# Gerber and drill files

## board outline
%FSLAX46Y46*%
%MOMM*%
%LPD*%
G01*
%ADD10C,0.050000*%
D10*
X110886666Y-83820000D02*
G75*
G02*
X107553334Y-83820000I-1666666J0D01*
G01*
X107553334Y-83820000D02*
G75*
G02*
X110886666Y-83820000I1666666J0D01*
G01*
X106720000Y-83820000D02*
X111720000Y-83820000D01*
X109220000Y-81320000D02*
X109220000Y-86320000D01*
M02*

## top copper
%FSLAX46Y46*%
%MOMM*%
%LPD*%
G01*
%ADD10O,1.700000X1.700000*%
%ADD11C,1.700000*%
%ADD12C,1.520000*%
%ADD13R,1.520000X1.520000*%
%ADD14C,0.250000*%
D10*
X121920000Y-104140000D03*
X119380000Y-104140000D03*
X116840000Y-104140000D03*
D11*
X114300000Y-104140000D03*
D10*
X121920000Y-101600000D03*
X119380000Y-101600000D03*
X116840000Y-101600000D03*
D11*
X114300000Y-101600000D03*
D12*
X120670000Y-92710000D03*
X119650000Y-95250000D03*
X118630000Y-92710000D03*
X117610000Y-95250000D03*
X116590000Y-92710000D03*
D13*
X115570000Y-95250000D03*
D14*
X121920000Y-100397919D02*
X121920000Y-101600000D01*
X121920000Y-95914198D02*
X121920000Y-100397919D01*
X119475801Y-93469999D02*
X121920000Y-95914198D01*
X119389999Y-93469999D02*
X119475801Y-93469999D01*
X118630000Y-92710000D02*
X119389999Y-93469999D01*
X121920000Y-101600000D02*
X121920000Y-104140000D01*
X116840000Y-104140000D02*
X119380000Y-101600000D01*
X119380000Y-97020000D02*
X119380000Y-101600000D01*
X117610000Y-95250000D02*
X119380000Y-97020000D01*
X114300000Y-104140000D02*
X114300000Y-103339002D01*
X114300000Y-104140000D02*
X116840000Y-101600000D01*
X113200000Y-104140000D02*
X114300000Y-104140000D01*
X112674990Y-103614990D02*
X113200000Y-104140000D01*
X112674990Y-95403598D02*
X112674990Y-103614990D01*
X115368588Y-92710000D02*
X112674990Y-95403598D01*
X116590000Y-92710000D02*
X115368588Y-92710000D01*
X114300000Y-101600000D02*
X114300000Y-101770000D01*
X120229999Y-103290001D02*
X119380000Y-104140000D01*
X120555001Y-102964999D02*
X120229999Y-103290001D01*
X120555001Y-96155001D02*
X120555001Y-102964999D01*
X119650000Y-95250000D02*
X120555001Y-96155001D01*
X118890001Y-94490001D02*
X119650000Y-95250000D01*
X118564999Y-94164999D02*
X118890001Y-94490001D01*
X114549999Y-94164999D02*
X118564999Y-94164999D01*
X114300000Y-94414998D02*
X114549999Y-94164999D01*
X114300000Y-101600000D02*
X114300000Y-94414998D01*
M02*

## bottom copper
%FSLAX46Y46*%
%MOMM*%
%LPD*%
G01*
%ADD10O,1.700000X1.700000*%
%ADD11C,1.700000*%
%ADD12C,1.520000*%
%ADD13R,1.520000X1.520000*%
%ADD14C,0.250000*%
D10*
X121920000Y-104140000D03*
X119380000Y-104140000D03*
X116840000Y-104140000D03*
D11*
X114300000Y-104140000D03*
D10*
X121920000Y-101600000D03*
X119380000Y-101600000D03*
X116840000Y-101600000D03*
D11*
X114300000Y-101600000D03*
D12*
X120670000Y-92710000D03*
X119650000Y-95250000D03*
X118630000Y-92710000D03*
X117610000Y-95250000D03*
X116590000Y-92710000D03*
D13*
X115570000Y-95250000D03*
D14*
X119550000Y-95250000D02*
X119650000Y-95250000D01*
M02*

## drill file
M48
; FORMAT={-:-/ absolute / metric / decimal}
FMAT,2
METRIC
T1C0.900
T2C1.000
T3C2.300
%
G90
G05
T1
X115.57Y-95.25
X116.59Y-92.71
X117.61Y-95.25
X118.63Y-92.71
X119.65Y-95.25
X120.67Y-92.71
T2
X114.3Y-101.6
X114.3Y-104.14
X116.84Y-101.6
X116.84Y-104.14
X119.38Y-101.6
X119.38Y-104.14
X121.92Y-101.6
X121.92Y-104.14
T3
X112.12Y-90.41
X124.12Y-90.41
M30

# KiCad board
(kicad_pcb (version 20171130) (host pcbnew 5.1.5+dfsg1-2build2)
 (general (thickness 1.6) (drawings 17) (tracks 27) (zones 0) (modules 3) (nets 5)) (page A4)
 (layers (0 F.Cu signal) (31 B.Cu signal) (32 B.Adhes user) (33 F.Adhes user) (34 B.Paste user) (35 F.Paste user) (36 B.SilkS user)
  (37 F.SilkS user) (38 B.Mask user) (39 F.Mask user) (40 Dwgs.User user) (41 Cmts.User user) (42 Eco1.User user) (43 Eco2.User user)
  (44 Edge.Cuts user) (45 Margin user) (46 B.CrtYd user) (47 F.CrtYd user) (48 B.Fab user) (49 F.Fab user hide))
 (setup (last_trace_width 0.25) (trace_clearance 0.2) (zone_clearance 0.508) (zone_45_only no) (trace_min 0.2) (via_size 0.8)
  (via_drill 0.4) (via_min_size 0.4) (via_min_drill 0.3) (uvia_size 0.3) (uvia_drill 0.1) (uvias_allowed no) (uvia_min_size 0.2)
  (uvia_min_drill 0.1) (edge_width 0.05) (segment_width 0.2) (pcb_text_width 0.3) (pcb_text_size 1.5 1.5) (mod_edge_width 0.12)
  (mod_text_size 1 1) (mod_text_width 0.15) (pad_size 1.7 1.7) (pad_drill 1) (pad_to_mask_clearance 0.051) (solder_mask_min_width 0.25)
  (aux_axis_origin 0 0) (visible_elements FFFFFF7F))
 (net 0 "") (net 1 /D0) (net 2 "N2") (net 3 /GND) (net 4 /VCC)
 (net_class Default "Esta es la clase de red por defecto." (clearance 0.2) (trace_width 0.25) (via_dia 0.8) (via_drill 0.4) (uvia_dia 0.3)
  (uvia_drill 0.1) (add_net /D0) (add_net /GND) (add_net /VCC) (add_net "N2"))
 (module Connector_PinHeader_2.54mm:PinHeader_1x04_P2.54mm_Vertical (layer F.Cu) (at 114.3 104.14 90)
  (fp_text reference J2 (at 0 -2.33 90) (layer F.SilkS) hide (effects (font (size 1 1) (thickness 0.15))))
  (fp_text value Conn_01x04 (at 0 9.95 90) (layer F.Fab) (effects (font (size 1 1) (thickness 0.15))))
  (pad 4 thru_hole oval (at 0 7.62 90) (size 1.7 1.7) (drill 1) (layers *.Cu *.Mask) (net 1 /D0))
  (pad 3 thru_hole oval (at 0 5.08 90) (size 1.7 1.7) (drill 1) (layers *.Cu *.Mask) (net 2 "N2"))
  (pad 2 thru_hole oval (at 0 2.54 90) (size 1.7 1.7) (drill 1) (layers *.Cu *.Mask) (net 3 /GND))
  (pad 1 thru_hole circle (at 0 0 90) (size 1.7 1.7) (drill 1) (layers *.Cu *.Mask) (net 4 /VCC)))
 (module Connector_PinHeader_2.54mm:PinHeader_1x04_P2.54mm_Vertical (layer F.Cu) (at 114.3 101.6 90)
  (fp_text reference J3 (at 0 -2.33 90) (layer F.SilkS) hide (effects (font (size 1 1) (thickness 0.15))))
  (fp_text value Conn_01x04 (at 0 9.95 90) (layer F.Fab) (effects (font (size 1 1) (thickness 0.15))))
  (pad 4 thru_hole oval (at 0 7.62 90) (size 1.7 1.7) (drill 1) (layers *.Cu *.Mask) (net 1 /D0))
  (pad 3 thru_hole oval (at 0 5.08 90) (size 1.7 1.7) (drill 1) (layers *.Cu *.Mask) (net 3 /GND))
  (pad 2 thru_hole oval (at 0 2.54 90) (size 1.7 1.7) (drill 1) (layers *.Cu *.Mask) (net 4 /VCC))
  (pad 1 thru_hole circle (at 0 0 90) (size 1.7 1.7) (drill 1) (layers *.Cu *.Mask) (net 2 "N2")))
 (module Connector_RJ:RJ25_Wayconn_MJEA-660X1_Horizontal (layer F.Cu) (at 115.57 95.25 180)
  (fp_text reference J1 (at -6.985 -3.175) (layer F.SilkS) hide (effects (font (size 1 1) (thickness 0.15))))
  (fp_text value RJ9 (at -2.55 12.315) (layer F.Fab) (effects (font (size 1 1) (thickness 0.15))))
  (pad "" np_thru_hole circle (at -8.55 4.84 180) (size 2.3 2.3) (drill 2.3) (layers *.Cu *.Mask))
  (pad "" np_thru_hole circle (at 3.45 4.84 180) (size 2.3 2.3) (drill 2.3) (layers *.Cu *.Mask))
  (pad 6 thru_hole circle (at -5.1 2.54 180) (size 1.52 1.52) (drill 0.9) (layers *.Cu *.Mask))
  (pad 5 thru_hole circle (at -4.08 0 180) (size 1.52 1.52) (drill 0.9) (layers *.Cu *.Mask) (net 2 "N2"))
  (pad 4 thru_hole circle (at -3.06 2.54 180) (size 1.52 1.52) (drill 0.9) (layers *.Cu *.Mask) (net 1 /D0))
  (pad 3 thru_hole circle (at -2.04 0 180) (size 1.52 1.52) (drill 0.9) (layers *.Cu *.Mask) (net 3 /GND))
  (pad 2 thru_hole circle (at -1.02 2.54 180) (size 1.52 1.52) (drill 0.9) (layers *.Cu *.Mask) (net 4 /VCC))
  (pad 1 thru_hole rect (at 0 0 180) (size 1.52 1.52) (drill 0.9) (layers *.Cu *.Mask)))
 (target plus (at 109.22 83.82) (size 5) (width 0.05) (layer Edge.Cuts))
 (segment (start 121.92 100.397919) (end 121.92 101.6) (width 0.25) (layer F.Cu) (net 1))
 (segment (start 121.92 95.914198) (end 121.92 100.397919) (width 0.25) (layer F.Cu) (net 1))
 (segment (start 119.475801 93.469999) (end 121.92 95.914198) (width 0.25) (layer F.Cu) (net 1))
 (segment (start 119.389999 93.469999) (end 119.475801 93.469999) (width 0.25) (layer F.Cu) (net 1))
 (segment (start 118.63 92.71) (end 119.389999 93.469999) (width 0.25) (layer F.Cu) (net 1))
 (segment (start 121.92 101.6) (end 121.92 104.14) (width 0.25) (layer F.Cu) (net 1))
 (segment (start 116.84 104.14) (end 119.38 101.6) (width 0.25) (layer F.Cu) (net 3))
 (segment (start 119.38 97.02) (end 119.38 101.6) (width 0.25) (layer F.Cu) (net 3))
 (segment (start 117.61 95.25) (end 119.38 97.02) (width 0.25) (layer F.Cu) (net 3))
 (segment (start 114.3 104.14) (end 114.3 103.339002) (width 0.25) (layer F.Cu) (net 4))
 (segment (start 114.3 104.14) (end 116.84 101.6) (width 0.25) (layer F.Cu) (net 4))
 (segment (start 113.2 104.14) (end 114.3 104.14) (width 0.25) (layer F.Cu) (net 4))
 (segment (start 112.67499 103.61499) (end 113.2 104.14) (width 0.25) (layer F.Cu) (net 4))
 (segment (start 112.67499 95.403598) (end 112.67499 103.61499) (width 0.25) (layer F.Cu) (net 4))
 (segment (start 115.368588 92.71) (end 112.67499 95.403598) (width 0.25) (layer F.Cu) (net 4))
 (segment (start 116.59 92.71) (end 115.368588 92.71) (width 0.25) (layer F.Cu) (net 4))
 (segment (start 114.3 101.6) (end 114.3 101.77) (width 0.25) (layer F.Cu) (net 2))
 (segment (start 120.229999 103.290001) (end 119.38 104.14) (width 0.25) (layer F.Cu) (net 2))
 (segment (start 120.555001 102.964999) (end 120.229999 103.290001) (width 0.25) (layer F.Cu) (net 2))
 (segment (start 120.555001 96.155001) (end 120.555001 102.964999) (width 0.25) (layer F.Cu) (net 2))
 (segment (start 119.65 95.25) (end 120.555001 96.155001) (width 0.25) (layer F.Cu) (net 2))
 (segment (start 119.55 95.25) (end 119.65 95.25) (width 0.25) (layer B.Cu) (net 2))
 (segment (start 118.890001 94.490001) (end 119.65 95.25) (width 0.25) (layer F.Cu) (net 2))
 (segment (start 118.564999 94.164999) (end 118.890001 94.490001) (width 0.25) (layer F.Cu) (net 2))
 (segment (start 114.549999 94.164999) (end 118.564999 94.164999) (width 0.25) (layer F.Cu) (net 2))
 (segment (start 114.3 94.414998) (end 114.549999 94.164999) (width 0.25) (layer F.Cu) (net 2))
 (segment (start 114.3 101.6) (end 114.3 94.414998) (width 0.25) (layer F.Cu) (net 2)))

